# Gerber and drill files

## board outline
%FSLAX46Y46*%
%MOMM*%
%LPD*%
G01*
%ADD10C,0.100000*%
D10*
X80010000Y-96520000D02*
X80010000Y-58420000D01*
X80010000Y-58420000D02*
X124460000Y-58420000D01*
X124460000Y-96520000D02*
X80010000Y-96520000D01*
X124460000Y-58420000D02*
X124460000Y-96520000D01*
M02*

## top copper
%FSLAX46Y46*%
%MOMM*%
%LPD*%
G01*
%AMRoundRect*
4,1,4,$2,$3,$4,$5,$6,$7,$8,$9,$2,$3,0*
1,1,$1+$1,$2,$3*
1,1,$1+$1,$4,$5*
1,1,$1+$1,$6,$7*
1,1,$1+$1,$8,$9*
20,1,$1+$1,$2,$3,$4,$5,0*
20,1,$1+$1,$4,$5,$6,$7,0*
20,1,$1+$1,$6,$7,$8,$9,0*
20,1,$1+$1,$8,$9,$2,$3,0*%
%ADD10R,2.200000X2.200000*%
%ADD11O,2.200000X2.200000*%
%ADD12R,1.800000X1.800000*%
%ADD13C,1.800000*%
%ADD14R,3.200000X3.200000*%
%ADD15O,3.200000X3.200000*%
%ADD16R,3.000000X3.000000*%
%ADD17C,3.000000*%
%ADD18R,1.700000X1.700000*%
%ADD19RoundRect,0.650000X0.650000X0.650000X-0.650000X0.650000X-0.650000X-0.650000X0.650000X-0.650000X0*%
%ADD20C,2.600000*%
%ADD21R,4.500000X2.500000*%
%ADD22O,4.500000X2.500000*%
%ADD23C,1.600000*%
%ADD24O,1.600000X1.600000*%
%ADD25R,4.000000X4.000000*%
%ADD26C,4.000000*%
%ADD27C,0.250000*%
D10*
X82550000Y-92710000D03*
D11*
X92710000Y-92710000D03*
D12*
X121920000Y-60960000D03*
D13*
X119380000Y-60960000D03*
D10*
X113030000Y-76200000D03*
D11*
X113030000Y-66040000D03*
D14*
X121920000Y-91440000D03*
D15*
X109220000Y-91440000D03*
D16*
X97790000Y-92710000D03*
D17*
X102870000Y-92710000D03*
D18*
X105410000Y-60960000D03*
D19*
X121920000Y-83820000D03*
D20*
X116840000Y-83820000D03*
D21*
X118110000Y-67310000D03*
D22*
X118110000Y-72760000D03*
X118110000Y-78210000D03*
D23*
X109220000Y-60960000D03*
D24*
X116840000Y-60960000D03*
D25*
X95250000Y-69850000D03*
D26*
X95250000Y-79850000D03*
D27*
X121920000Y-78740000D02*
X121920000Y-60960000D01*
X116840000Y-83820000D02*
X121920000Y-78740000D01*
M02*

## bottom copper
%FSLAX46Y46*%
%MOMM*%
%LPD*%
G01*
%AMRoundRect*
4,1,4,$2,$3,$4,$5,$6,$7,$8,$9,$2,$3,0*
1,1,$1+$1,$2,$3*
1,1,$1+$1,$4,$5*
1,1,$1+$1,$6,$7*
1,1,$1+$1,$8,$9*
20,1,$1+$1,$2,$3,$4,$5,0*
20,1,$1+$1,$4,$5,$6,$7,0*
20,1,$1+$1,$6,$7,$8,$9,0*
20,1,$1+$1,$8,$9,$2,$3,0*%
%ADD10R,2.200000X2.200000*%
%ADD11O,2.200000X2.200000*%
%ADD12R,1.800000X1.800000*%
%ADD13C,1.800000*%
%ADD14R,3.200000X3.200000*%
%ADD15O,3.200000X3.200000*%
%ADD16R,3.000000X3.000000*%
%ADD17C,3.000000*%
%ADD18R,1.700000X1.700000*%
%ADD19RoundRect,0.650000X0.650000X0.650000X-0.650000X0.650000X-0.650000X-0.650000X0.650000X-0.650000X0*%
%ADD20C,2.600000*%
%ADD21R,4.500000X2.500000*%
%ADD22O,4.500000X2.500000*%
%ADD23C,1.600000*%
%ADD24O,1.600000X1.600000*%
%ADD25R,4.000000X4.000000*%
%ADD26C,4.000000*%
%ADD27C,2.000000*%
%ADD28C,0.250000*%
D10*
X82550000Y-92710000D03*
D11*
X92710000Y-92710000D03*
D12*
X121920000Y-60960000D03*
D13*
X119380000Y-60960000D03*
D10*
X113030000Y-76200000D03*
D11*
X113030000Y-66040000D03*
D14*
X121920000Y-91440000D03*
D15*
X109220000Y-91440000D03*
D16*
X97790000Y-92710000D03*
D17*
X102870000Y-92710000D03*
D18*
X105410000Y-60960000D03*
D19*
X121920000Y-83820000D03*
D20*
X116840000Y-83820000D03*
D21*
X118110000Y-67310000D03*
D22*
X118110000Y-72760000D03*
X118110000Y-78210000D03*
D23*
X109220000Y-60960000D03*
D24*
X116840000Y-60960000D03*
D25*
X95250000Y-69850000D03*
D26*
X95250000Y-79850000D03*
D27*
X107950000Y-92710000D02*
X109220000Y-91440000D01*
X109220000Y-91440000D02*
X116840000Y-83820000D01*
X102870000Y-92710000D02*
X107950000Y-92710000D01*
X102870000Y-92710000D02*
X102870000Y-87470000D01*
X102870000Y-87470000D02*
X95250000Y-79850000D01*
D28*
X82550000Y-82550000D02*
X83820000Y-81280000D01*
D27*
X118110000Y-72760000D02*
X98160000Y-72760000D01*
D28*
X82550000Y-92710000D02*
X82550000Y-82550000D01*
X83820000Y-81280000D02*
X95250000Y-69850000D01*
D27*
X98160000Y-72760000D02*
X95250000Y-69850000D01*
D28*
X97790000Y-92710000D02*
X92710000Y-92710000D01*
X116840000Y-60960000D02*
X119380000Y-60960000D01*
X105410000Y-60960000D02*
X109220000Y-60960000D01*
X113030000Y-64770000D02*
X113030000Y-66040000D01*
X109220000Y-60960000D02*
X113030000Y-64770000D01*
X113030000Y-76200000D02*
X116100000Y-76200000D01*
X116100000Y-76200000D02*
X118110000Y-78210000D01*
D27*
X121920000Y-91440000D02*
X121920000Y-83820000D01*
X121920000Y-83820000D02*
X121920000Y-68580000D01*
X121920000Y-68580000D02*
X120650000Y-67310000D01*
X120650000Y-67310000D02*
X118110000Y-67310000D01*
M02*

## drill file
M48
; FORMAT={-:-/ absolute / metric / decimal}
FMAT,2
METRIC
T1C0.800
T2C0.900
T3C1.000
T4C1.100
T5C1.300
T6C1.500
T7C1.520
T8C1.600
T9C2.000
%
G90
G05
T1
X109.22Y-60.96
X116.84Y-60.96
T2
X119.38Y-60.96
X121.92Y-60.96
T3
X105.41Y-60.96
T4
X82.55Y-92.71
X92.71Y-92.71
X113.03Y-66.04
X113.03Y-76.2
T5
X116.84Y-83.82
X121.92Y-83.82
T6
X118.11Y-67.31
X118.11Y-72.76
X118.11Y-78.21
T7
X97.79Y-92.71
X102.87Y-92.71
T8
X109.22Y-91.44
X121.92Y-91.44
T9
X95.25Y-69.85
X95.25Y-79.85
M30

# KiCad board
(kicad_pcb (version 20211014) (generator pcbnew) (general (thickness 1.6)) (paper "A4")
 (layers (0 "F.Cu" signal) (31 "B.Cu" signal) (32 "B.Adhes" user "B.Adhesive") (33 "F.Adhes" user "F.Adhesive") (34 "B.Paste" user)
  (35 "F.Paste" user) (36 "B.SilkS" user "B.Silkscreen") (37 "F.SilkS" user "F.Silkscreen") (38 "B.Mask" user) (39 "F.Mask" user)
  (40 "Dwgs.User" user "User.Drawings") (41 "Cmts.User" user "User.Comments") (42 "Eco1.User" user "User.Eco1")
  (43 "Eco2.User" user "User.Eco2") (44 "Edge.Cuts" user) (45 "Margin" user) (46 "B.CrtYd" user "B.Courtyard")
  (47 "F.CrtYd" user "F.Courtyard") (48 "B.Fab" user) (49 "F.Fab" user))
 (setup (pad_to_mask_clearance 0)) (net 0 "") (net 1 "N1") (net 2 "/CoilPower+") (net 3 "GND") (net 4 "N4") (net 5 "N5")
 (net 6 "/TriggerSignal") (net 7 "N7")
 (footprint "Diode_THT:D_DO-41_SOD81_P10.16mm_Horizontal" (layer "F.Cu") (at 82.55 92.71)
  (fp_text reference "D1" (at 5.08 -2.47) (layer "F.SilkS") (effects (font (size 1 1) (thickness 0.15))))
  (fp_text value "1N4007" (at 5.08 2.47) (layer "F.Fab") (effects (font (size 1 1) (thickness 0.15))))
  (pad "1" thru_hole rect (at 0 0) (size 2.2 2.2) (drill 1.1) (layers *.Cu *.Mask) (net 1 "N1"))
  (pad "2" thru_hole oval (at 10.16 0) (size 2.2 2.2) (drill 1.1) (layers *.Cu *.Mask) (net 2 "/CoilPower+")))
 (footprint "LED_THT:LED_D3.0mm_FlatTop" (layer "F.Cu") (at 121.92 60.96 180)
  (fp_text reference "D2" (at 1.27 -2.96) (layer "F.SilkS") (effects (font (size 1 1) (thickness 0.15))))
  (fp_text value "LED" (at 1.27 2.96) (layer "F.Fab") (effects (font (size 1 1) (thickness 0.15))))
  (pad "1" thru_hole rect (at 0 0 180) (size 1.8 1.8) (drill 0.9) (layers *.Cu *.Mask) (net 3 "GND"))
  (pad "2" thru_hole circle (at 2.54 0 180) (size 1.8 1.8) (drill 0.9) (layers *.Cu *.Mask) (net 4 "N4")))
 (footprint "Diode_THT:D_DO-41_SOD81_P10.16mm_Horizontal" (layer "F.Cu") (at 113.03 76.2 90)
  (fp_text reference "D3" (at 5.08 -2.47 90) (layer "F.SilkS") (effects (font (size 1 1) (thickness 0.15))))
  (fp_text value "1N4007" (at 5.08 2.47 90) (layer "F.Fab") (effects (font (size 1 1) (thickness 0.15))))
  (pad "1" thru_hole rect (at 0 0 90) (size 2.2 2.2) (drill 1.1) (layers *.Cu *.Mask) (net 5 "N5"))
  (pad "2" thru_hole oval (at 10.16 0 90) (size 2.2 2.2) (drill 1.1) (layers *.Cu *.Mask) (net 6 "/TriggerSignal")))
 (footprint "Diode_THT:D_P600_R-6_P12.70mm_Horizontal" (layer "F.Cu") (at 121.92 91.44 180)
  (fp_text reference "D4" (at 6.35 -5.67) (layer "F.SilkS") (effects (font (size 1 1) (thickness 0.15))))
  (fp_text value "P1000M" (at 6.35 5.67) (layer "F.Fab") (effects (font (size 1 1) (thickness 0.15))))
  (pad "1" thru_hole rect (at 0 0 180) (size 3.2 3.2) (drill 1.6) (layers *.Cu *.Mask) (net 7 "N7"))
  (pad "2" thru_hole oval (at 12.7 0 180) (size 3.2 3.2) (drill 1.6) (layers *.Cu *.Mask) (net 3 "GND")))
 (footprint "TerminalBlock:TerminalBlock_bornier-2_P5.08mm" (layer "F.Cu") (at 97.79 92.71)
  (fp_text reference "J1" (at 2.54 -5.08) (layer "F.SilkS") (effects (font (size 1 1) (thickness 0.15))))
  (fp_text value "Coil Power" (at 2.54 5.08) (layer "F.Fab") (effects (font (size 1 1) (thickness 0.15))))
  (pad "1" thru_hole rect (at 0 0) (size 3 3) (drill 1.52) (layers *.Cu *.Mask) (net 2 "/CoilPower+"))
  (pad "2" thru_hole circle (at 5.08 0) (size 3 3) (drill 1.52) (layers *.Cu *.Mask) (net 3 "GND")))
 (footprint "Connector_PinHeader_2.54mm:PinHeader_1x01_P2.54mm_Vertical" (layer "F.Cu") (at 105.41 60.96)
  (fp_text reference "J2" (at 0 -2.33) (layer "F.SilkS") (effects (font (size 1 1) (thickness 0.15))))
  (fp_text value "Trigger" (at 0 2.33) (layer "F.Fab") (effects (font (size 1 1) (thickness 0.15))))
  (pad "1" thru_hole rect (at 0 0) (size 1.7 1.7) (drill 1) (layers *.Cu *.Mask) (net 6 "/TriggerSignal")))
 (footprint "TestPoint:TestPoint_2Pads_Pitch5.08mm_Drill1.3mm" (layer "F.Cu") (at 121.92 83.82 180)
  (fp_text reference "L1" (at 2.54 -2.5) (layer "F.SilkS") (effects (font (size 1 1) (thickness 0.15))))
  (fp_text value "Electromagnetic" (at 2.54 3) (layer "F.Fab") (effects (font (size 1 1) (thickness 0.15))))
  (pad "1" thru_hole roundrect (at 0 0 180) (size 2.6 2.6) (drill 1.3) (layers *.Cu *.Mask) (roundrect_rratio 0.25) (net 7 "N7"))
  (pad "2" thru_hole circle (at 5.08 0 180) (size 2.6 2.6) (drill 1.3) (layers *.Cu *.Mask) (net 3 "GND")))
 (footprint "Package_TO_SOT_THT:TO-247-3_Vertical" (layer "F.Cu") (at 118.11 67.31 -90)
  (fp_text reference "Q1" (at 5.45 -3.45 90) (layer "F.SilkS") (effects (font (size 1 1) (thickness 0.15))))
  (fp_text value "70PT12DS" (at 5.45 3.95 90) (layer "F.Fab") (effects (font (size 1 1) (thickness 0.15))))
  (pad "1" thru_hole rect (at 0 0 270) (size 2.5 4.5) (drill 1.5) (layers *.Cu *.Mask) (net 7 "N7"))
  (pad "2" thru_hole oval (at 5.45 0 270) (size 2.5 4.5) (drill 1.5) (layers *.Cu *.Mask) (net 1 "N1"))
  (pad "3" thru_hole oval (at 10.9 0 270) (size 2.5 4.5) (drill 1.5) (layers *.Cu *.Mask) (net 5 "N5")))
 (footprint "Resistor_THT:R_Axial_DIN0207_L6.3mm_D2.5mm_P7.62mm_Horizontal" (layer "F.Cu") (at 109.22 60.96)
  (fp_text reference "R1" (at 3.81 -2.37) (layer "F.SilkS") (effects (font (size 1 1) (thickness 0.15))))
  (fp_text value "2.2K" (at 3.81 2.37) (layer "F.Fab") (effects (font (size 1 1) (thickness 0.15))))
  (pad "1" thru_hole circle (at 0 0) (size 1.6 1.6) (drill 0.8) (layers *.Cu *.Mask) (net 6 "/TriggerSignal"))
  (pad "2" thru_hole oval (at 7.62 0) (size 1.6 1.6) (drill 0.8) (layers *.Cu *.Mask) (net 4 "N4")))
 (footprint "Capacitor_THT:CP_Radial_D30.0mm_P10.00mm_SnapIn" (layer "B.Cu") (at 95.25 69.85 -90)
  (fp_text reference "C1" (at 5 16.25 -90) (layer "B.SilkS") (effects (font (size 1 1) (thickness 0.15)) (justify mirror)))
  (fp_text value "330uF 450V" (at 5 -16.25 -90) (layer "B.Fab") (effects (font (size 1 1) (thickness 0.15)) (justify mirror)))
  (pad "1" thru_hole rect (at 0 0 270) (size 4 4) (drill 2) (layers *.Cu *.Mask) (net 1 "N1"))
  (pad "2" thru_hole circle (at 10 0 270) (size 4 4) (drill 2) (layers *.Cu *.Mask) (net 3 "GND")))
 (gr_line (start 80.01 96.52) (end 80.01 58.42) (layer "Edge.Cuts") (width 0.1))
 (gr_line (start 80.01 58.42) (end 124.46 58.42) (layer "Edge.Cuts") (width 0.1))
 (gr_line (start 124.46 96.52) (end 80.01 96.52) (layer "Edge.Cuts") (width 0.1))
 (gr_line (start 124.46 58.42) (end 124.46 96.52) (layer "Edge.Cuts") (width 0.1))
 (segment (start 121.92 78.74) (end 121.92 60.96) (width 0.25) (layer "F.Cu") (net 3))
 (segment (start 116.84 83.82) (end 121.92 78.74) (width 0.25) (layer "F.Cu") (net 3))
 (segment (start 107.95 92.71) (end 109.22 91.44) (width 2) (layer "B.Cu") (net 3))
 (segment (start 109.22 91.44) (end 116.84 83.82) (width 2) (layer "B.Cu") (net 3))
 (segment (start 102.87 92.71) (end 107.95 92.71) (width 2) (layer "B.Cu") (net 3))
 (segment (start 102.87 92.71) (end 102.87 87.47) (width 2) (layer "B.Cu") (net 3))
 (segment (start 102.87 87.47) (end 95.25 79.85) (width 2) (layer "B.Cu") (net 3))
 (segment (start 82.55 82.55) (end 83.82 81.28) (width 0.25) (layer "B.Cu") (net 1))
 (segment (start 118.11 72.76) (end 98.16 72.76) (width 2) (layer "B.Cu") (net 1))
 (segment (start 82.55 92.71) (end 82.55 82.55) (width 0.25) (layer "B.Cu") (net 1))
 (segment (start 83.82 81.28) (end 95.25 69.85) (width 0.25) (layer "B.Cu") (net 1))
 (segment (start 98.16 72.76) (end 95.25 69.85) (width 2) (layer "B.Cu") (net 1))
 (segment (start 97.79 92.71) (end 92.71 92.71) (width 0.25) (layer "B.Cu") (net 2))
 (segment (start 116.84 60.96) (end 119.38 60.96) (width 0.25) (layer "B.Cu") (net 4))
 (segment (start 105.41 60.96) (end 109.22 60.96) (width 0.25) (layer "B.Cu") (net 6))
 (segment (start 113.03 64.77) (end 113.03 66.04) (width 0.25) (layer "B.Cu") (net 6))
 (segment (start 109.22 60.96) (end 113.03 64.77) (width 0.25) (layer "B.Cu") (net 6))
 (segment (start 113.03 76.2) (end 116.1 76.2) (width 0.25) (layer "B.Cu") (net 5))
 (segment (start 116.1 76.2) (end 118.11 78.21) (width 0.25) (layer "B.Cu") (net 5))
 (segment (start 121.92 91.44) (end 121.92 83.82) (width 2) (layer "B.Cu") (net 7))
 (segment (start 121.92 83.82) (end 121.92 68.58) (width 2) (layer "B.Cu") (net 7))
 (segment (start 121.92 68.58) (end 120.65 67.31) (width 2) (layer "B.Cu") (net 7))
 (segment (start 120.65 67.31) (end 118.11 67.31) (width 2) (layer "B.Cu") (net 7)))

